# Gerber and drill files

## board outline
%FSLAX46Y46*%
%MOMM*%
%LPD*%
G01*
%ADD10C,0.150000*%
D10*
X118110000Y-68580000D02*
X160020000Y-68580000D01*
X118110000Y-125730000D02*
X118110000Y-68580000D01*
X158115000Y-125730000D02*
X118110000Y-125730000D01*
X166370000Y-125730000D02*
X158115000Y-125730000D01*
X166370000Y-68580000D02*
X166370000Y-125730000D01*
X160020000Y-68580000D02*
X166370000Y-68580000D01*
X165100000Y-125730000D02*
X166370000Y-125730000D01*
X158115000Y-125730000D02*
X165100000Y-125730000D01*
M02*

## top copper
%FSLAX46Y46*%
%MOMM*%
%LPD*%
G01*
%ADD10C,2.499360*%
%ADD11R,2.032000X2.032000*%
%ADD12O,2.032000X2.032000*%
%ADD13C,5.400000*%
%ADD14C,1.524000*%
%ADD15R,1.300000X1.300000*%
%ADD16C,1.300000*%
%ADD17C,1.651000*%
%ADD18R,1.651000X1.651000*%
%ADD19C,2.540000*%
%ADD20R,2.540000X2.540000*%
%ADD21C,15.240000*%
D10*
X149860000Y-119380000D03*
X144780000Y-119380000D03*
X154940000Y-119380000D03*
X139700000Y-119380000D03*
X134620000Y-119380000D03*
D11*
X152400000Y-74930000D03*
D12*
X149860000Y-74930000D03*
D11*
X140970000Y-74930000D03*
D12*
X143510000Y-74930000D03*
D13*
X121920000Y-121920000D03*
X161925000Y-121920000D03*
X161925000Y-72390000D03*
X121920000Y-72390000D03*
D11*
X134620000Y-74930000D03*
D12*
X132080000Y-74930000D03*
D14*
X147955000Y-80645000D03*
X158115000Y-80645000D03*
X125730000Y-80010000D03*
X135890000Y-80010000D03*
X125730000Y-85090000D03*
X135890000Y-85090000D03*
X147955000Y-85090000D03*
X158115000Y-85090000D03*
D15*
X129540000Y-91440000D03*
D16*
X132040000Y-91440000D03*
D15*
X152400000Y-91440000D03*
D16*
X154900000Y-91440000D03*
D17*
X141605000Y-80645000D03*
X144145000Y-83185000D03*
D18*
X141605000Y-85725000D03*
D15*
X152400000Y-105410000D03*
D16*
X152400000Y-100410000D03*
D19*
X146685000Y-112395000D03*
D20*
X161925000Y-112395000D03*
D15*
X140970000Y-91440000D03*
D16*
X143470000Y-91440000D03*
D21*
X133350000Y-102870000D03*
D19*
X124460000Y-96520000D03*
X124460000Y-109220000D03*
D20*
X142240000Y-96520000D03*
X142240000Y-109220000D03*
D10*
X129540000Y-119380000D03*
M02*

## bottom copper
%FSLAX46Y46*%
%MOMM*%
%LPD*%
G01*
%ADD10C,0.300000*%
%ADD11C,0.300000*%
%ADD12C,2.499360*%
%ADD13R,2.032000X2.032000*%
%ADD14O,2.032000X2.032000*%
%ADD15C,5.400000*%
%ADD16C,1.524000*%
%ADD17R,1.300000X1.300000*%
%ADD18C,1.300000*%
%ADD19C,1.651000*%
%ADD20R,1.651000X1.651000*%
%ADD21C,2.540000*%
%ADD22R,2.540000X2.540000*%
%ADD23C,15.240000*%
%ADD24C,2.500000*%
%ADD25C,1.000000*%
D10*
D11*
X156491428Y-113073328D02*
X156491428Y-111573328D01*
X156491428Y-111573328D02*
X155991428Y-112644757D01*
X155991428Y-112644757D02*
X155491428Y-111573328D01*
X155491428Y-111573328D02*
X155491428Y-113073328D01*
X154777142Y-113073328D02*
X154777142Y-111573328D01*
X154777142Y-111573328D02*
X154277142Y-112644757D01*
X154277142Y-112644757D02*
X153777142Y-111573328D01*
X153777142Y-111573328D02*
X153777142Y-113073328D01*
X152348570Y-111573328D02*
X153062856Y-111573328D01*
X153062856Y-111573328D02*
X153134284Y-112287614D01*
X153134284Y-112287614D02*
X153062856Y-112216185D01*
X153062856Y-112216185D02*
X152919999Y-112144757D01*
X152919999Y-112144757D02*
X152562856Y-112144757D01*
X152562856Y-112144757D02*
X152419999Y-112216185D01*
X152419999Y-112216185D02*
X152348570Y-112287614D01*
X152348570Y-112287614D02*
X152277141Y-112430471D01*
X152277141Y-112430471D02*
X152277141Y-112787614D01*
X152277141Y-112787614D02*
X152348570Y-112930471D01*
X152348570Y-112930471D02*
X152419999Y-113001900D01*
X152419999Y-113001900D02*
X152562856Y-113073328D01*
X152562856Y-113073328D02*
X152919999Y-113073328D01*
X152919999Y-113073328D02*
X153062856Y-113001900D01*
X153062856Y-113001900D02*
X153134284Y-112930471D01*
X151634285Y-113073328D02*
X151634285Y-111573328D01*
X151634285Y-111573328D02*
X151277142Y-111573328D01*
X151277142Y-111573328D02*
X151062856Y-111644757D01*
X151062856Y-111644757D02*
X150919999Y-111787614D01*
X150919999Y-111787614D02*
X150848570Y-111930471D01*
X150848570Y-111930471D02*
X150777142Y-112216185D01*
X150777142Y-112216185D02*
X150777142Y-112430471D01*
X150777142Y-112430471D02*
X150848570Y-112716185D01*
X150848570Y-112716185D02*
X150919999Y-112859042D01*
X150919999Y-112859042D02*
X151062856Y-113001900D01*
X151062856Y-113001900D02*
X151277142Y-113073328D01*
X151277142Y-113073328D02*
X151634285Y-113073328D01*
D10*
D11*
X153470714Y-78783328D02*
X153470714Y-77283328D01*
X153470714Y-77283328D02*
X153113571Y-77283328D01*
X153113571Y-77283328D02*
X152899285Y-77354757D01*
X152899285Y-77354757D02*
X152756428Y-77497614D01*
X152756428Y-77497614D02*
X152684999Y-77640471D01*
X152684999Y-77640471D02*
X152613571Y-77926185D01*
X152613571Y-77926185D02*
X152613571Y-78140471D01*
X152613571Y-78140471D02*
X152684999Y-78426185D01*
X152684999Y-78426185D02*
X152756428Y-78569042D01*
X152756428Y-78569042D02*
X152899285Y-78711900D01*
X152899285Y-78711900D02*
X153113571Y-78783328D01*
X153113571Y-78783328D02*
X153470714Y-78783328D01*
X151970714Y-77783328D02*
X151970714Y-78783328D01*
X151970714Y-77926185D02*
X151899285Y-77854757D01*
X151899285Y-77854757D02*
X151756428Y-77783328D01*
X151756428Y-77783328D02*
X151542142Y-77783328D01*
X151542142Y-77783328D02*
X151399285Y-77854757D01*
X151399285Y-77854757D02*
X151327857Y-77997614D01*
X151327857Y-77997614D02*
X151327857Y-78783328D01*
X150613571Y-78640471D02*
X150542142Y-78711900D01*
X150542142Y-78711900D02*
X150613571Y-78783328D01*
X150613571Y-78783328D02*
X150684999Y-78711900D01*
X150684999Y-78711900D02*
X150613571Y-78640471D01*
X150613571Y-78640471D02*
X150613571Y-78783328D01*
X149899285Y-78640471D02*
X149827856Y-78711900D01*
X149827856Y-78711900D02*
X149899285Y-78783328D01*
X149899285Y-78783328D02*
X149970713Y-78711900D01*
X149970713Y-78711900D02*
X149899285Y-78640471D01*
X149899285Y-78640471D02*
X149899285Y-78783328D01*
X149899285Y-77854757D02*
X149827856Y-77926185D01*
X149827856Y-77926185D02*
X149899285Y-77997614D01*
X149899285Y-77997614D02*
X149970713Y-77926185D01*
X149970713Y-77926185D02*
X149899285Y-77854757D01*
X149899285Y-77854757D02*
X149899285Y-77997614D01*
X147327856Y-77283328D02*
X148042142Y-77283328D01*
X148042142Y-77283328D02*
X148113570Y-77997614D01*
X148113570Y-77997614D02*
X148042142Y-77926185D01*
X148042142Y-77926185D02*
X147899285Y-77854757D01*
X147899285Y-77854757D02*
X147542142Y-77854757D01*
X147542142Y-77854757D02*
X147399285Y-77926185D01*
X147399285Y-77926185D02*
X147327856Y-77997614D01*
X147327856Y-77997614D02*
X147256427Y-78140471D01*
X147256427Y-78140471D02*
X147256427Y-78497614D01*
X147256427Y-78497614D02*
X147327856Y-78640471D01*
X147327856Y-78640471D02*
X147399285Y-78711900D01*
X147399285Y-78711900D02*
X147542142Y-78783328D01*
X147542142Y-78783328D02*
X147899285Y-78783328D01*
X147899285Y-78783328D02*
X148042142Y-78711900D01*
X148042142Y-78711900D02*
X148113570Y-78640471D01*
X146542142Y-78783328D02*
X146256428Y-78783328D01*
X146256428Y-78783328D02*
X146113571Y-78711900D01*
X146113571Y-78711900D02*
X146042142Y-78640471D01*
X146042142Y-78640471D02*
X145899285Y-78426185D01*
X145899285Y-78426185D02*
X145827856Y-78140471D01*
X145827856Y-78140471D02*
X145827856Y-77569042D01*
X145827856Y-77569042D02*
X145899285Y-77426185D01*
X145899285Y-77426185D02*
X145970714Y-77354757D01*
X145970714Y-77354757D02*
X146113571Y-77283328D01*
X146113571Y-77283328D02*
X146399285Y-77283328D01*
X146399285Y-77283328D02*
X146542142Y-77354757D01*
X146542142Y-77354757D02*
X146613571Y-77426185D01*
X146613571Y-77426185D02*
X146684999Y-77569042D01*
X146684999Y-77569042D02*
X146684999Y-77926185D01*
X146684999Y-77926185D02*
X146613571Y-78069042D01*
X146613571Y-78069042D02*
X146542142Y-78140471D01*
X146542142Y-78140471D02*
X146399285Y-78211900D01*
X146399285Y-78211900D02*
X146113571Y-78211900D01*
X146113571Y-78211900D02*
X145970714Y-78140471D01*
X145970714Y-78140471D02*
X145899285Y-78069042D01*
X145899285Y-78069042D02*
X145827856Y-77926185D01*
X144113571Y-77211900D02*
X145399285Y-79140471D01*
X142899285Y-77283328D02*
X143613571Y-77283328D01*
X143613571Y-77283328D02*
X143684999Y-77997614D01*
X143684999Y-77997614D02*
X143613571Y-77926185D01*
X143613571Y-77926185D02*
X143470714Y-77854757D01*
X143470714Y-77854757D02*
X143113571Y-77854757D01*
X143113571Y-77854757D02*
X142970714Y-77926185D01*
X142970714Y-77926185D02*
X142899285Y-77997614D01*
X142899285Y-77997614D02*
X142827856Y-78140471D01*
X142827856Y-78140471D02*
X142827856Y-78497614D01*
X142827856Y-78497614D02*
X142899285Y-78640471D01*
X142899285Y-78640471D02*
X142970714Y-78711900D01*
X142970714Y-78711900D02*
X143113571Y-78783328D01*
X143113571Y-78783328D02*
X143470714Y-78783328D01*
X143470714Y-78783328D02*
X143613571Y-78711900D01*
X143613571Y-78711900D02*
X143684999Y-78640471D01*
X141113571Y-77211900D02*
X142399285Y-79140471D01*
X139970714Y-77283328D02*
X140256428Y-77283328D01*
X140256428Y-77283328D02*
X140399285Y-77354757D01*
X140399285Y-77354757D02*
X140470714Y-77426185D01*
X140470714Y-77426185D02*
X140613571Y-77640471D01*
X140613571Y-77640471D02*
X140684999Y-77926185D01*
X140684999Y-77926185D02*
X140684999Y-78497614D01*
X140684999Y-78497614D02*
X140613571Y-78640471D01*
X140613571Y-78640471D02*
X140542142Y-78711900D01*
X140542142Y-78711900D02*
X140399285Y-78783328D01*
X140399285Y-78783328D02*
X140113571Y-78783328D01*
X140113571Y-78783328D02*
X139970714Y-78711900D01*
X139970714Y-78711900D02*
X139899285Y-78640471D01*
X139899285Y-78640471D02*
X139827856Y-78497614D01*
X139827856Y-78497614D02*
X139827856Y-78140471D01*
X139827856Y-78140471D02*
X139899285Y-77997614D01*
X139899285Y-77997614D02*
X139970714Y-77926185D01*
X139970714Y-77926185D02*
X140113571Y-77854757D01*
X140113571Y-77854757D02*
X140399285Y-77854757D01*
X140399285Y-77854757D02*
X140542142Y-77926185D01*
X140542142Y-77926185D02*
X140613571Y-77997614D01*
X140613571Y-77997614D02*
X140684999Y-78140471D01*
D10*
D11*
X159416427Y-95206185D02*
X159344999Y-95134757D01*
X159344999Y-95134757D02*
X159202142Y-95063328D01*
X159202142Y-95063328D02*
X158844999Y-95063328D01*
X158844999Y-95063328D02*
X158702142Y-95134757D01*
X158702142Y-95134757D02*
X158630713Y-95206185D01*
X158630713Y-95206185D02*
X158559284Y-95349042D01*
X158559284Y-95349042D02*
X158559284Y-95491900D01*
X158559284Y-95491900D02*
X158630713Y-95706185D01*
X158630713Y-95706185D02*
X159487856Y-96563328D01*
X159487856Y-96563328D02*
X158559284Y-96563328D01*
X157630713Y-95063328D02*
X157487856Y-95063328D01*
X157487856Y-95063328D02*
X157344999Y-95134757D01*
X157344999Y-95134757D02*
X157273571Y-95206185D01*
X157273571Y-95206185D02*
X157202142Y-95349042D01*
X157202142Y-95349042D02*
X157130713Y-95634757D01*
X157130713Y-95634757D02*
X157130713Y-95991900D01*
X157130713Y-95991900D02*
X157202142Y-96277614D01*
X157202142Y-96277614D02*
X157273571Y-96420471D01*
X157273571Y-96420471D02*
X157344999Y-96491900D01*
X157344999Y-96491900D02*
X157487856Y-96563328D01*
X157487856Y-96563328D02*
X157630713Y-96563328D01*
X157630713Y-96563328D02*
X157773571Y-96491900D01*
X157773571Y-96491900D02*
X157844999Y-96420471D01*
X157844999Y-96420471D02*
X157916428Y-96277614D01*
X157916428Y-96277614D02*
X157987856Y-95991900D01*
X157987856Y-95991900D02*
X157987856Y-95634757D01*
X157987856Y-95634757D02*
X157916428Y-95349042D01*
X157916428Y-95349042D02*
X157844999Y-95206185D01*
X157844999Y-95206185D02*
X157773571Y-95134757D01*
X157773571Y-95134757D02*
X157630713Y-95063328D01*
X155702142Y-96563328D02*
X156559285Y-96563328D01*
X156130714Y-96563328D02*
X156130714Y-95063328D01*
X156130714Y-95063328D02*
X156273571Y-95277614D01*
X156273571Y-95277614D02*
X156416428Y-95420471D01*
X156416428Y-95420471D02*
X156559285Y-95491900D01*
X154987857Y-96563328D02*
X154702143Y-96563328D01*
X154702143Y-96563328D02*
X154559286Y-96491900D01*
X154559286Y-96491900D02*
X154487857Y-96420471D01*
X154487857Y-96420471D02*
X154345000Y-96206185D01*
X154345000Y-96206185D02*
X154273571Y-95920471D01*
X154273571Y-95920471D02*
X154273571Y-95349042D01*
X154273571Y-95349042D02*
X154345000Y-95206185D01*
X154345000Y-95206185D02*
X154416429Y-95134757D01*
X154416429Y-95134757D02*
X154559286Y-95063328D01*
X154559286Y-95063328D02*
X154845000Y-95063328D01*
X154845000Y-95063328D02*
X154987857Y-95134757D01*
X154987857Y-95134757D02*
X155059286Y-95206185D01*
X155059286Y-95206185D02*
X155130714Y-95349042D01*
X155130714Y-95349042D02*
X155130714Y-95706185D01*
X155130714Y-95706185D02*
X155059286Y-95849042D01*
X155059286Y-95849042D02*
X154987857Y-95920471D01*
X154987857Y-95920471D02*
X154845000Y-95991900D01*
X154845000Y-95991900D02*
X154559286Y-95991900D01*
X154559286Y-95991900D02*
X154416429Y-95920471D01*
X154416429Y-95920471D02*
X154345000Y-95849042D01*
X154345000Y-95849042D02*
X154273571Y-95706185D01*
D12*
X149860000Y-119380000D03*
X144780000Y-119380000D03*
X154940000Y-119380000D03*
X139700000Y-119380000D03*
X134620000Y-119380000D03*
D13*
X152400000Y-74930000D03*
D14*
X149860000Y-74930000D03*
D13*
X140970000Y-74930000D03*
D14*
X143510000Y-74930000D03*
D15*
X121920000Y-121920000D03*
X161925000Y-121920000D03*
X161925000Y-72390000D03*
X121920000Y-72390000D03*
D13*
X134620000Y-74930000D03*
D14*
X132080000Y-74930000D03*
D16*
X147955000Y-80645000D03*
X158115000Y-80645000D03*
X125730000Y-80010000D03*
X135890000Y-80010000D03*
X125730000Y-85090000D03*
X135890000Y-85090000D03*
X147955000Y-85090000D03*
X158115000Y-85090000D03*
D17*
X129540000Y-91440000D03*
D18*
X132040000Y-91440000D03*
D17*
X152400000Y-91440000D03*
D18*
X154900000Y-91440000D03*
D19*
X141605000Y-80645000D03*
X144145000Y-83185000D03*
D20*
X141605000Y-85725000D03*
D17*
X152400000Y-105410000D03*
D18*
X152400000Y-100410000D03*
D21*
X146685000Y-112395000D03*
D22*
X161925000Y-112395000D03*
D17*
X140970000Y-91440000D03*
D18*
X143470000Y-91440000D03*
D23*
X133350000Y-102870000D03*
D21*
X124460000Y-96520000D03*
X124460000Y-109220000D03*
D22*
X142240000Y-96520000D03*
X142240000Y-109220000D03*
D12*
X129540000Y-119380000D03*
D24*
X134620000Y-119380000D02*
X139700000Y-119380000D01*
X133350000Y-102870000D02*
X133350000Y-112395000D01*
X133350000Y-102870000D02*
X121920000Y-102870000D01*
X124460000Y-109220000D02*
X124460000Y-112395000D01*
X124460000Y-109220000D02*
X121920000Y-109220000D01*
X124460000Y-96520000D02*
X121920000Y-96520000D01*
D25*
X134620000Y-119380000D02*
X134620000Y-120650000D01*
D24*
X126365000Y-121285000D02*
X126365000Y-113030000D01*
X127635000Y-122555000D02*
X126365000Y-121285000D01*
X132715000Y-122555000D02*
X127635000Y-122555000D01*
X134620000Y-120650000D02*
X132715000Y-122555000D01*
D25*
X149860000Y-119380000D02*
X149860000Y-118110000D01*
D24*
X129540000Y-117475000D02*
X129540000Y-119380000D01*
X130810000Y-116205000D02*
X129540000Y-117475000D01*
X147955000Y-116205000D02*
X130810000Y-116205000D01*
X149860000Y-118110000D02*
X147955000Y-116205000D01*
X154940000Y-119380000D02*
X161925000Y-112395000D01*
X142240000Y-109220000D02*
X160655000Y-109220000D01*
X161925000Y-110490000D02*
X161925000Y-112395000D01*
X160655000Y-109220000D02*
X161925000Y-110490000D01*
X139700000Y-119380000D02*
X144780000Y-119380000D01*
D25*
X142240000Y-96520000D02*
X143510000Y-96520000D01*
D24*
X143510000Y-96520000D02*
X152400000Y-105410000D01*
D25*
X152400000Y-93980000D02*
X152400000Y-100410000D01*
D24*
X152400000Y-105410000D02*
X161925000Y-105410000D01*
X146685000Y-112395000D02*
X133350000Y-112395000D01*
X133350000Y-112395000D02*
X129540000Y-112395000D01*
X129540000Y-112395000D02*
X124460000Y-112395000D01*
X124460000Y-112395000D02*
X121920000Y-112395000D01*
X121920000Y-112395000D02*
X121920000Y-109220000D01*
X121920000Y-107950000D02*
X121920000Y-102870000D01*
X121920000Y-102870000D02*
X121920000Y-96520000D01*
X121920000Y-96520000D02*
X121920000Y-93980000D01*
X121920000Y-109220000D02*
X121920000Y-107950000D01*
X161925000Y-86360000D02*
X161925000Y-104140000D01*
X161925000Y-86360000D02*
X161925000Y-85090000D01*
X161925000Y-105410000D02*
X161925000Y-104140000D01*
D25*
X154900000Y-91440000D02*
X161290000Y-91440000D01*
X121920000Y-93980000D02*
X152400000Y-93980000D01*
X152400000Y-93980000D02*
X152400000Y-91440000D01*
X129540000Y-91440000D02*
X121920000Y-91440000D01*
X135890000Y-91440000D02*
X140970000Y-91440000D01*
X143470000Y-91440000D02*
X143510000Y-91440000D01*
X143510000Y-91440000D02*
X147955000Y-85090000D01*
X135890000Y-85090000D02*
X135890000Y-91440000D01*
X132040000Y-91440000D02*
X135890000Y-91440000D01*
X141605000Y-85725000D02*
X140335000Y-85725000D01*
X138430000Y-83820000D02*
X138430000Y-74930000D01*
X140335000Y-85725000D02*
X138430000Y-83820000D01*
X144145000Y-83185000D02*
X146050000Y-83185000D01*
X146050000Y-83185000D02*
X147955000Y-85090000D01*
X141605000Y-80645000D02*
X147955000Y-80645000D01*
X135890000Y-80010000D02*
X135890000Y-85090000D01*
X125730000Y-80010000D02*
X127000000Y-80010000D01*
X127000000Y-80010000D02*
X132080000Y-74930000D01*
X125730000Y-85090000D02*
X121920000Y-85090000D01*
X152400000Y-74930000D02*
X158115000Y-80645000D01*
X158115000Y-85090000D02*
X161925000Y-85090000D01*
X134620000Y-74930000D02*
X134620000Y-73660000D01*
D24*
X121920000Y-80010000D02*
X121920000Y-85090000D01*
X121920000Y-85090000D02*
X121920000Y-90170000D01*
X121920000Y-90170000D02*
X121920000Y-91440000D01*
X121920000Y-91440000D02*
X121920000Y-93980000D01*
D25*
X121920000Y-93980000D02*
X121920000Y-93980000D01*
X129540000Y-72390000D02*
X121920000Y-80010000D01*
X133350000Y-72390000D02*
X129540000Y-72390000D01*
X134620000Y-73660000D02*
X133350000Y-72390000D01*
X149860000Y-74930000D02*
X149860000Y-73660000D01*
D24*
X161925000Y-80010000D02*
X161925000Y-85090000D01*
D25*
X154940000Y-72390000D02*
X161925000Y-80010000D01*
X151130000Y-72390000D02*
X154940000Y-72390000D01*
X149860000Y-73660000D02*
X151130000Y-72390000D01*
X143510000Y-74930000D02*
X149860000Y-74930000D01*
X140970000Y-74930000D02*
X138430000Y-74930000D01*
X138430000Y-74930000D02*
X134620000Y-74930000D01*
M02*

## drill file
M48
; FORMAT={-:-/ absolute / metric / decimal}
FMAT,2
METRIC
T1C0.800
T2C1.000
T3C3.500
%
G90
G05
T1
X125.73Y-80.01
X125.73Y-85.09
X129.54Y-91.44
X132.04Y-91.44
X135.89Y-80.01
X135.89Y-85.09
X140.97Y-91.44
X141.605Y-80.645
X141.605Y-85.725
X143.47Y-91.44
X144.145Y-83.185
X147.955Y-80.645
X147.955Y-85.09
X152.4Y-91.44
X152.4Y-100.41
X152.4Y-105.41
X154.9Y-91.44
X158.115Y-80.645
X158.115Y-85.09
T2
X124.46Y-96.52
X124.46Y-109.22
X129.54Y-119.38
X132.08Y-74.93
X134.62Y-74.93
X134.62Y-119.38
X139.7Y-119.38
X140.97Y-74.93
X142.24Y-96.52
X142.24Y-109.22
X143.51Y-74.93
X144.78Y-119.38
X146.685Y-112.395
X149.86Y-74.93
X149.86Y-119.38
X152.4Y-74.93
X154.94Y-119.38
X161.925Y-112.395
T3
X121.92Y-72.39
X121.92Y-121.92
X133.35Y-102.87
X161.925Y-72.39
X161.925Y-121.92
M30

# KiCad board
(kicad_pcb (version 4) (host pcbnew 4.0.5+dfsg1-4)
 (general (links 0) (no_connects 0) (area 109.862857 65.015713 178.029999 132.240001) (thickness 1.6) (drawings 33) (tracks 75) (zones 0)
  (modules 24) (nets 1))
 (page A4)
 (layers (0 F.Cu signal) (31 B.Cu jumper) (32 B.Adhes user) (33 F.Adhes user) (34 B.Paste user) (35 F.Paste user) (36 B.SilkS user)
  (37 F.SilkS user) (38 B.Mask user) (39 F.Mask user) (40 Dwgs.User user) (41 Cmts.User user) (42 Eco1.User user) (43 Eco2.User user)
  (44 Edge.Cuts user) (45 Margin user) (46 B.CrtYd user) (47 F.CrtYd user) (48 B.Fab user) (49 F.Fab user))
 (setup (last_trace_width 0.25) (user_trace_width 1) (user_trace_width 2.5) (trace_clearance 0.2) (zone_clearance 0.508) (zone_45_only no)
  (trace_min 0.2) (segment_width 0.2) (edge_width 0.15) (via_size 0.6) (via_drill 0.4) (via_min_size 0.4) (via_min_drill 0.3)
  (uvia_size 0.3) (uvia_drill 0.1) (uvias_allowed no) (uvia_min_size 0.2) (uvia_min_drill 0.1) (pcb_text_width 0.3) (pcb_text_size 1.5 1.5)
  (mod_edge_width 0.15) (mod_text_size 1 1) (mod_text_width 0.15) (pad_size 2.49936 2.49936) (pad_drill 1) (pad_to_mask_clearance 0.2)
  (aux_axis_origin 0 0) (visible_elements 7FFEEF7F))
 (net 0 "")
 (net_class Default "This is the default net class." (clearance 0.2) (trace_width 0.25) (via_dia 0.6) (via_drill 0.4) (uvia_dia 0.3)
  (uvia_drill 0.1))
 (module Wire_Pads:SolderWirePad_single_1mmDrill (layer F.Cu) (at 149.86 119.38)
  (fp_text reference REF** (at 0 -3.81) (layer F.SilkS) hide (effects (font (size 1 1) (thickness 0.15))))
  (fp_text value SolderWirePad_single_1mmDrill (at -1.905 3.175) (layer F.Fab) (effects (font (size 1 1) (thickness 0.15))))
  (pad 2 thru_hole circle (at 0 0) (size 2.49936 2.49936) (drill 1) (layers *.Cu *.Mask)))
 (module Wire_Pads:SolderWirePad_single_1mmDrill (layer F.Cu) (at 144.78 119.38)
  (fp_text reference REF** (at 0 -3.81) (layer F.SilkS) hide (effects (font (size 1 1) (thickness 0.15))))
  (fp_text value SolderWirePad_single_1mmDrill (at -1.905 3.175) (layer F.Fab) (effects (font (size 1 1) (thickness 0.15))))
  (pad 1 thru_hole circle (at 0 0) (size 2.49936 2.49936) (drill 1) (layers *.Cu *.Mask)))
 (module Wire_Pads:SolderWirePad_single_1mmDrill (layer F.Cu) (at 154.94 119.38)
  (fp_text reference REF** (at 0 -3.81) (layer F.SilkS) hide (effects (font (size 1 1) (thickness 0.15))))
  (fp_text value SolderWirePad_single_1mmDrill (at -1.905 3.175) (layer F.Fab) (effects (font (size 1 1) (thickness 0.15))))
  (pad 3 thru_hole circle (at 0 0) (size 2.49936 2.49936) (drill 1) (layers *.Cu *.Mask)))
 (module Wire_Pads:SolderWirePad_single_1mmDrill (layer F.Cu) (at 139.7 119.38)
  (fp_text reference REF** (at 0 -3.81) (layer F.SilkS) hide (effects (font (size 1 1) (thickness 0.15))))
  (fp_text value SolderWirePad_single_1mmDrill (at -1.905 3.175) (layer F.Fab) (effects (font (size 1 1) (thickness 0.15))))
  (pad 3 thru_hole circle (at 0 0) (size 2.49936 2.49936) (drill 1) (layers *.Cu *.Mask)))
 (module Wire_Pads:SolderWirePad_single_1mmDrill (layer F.Cu) (at 134.62 119.38)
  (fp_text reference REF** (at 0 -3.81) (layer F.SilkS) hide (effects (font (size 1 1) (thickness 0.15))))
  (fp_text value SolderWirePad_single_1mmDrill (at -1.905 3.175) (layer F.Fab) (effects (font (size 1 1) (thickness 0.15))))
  (pad 2 thru_hole circle (at 0 0) (size 2.49936 2.49936) (drill 1) (layers *.Cu *.Mask)))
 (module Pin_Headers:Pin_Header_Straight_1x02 (layer F.Cu) (at 152.4 74.93 270)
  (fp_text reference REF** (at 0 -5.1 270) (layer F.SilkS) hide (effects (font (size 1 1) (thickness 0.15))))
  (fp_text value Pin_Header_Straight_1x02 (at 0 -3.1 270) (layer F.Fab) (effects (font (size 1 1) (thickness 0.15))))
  (pad 1 thru_hole rect (at 0 0 270) (size 2.032 2.032) (drill 1) (layers *.Cu *.Mask))
  (pad 2 thru_hole oval (at 0 2.54 270) (size 2.032 2.032) (drill 1) (layers *.Cu *.Mask)))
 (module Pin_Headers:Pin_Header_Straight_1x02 (layer F.Cu) (at 140.97 74.93 90)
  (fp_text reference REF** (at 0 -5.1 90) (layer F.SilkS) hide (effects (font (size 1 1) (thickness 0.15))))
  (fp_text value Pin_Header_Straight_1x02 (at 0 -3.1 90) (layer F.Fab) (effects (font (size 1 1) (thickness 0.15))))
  (pad 1 thru_hole rect (at 0 0 90) (size 2.032 2.032) (drill 1) (layers *.Cu *.Mask))
  (pad 2 thru_hole oval (at 0 2.54 90) (size 2.032 2.032) (drill 1) (layers *.Cu *.Mask)))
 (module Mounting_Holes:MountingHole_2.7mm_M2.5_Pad (layer F.Cu) (at 121.92 121.92)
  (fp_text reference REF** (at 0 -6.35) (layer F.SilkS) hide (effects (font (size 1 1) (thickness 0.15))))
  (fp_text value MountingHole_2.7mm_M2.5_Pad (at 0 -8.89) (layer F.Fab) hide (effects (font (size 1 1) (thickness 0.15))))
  (pad 1 thru_hole circle (at 0 0) (size 5.4 5.4) (drill 3.5) (layers *.Cu *.Mask)))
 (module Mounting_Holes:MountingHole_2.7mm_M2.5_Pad (layer F.Cu) (at 161.925 121.92)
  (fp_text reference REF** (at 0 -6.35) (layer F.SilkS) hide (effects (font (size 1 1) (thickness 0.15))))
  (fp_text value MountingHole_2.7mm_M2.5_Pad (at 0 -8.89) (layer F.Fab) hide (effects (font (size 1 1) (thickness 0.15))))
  (pad 1 thru_hole circle (at 0 0) (size 5.4 5.4) (drill 3.5) (layers *.Cu *.Mask)))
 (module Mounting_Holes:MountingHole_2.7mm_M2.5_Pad (layer F.Cu) (at 161.925 72.39)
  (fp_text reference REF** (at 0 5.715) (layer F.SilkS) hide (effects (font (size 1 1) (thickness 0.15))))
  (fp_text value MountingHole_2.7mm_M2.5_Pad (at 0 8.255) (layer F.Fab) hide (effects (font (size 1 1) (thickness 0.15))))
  (pad 1 thru_hole circle (at 0 0) (size 5.4 5.4) (drill 3.5) (layers *.Cu *.Mask)))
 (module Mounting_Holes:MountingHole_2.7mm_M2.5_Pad (layer F.Cu) (at 121.92 72.39)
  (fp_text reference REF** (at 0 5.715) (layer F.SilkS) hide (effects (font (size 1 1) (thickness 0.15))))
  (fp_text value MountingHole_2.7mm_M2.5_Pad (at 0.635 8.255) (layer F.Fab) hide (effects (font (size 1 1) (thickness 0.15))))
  (pad 1 thru_hole circle (at 0 0) (size 5.4 5.4) (drill 3.5) (layers *.Cu *.Mask)))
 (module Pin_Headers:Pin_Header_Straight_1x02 (layer F.Cu) (at 134.62 74.93 270)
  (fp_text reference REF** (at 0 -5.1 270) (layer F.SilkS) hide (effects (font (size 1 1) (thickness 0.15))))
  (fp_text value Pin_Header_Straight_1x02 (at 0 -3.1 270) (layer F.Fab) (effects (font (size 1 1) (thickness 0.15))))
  (pad 1 thru_hole rect (at 0 0 270) (size 2.032 2.032) (drill 1) (layers *.Cu *.Mask))
  (pad 2 thru_hole oval (at 0 2.54 270) (size 2.032 2.032) (drill 1) (layers *.Cu *.Mask)))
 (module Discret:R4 (layer F.Cu) (at 153.035 80.645)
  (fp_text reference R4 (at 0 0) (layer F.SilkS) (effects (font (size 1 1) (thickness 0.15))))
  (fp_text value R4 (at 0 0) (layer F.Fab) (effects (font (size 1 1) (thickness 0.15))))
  (pad 1 thru_hole circle (at -5.08 0) (size 1.524 1.524) (drill 0.8) (layers *.Cu *.Mask))
  (pad 2 thru_hole circle (at 5.08 0) (size 1.524 1.524) (drill 0.8) (layers *.Cu *.Mask)))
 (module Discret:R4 (layer F.Cu) (at 130.81 80.01)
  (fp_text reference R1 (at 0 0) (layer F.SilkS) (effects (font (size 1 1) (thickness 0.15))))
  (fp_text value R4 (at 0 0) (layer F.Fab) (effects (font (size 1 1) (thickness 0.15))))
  (pad 1 thru_hole circle (at -5.08 0) (size 1.524 1.524) (drill 0.8) (layers *.Cu *.Mask))
  (pad 2 thru_hole circle (at 5.08 0) (size 1.524 1.524) (drill 0.8) (layers *.Cu *.Mask)))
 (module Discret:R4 (layer F.Cu) (at 130.81 85.09)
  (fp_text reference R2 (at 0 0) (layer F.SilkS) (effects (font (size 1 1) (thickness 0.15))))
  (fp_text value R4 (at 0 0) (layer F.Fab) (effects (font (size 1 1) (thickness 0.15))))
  (pad 1 thru_hole circle (at -5.08 0) (size 1.524 1.524) (drill 0.8) (layers *.Cu *.Mask))
  (pad 2 thru_hole circle (at 5.08 0) (size 1.524 1.524) (drill 0.8) (layers *.Cu *.Mask)))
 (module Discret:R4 (layer F.Cu) (at 153.035 85.09)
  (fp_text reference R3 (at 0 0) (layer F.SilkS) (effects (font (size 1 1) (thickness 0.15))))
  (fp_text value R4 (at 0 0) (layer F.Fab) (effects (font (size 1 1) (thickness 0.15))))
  (pad 1 thru_hole circle (at -5.08 0) (size 1.524 1.524) (drill 0.8) (layers *.Cu *.Mask))
  (pad 2 thru_hole circle (at 5.08 0) (size 1.524 1.524) (drill 0.8) (layers *.Cu *.Mask)))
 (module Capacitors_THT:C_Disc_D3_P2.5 (layer F.Cu) (at 129.54 91.44)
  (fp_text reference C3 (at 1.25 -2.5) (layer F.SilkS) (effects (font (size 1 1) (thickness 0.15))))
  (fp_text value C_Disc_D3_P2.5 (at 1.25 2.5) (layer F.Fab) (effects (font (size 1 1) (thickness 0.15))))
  (pad 1 thru_hole rect (at 0 0) (size 1.3 1.3) (drill 0.8) (layers *.Cu *.Mask))
  (pad 2 thru_hole circle (at 2.5 0) (size 1.3 1.3) (drill 0.8) (layers *.Cu *.Mask)))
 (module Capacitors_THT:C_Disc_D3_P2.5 (layer F.Cu) (at 152.4 91.44)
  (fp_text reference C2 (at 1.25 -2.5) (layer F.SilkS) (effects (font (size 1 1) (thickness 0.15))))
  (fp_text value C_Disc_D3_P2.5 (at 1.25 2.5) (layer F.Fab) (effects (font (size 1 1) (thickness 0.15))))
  (pad 1 thru_hole rect (at 0 0) (size 1.3 1.3) (drill 0.8) (layers *.Cu *.Mask))
  (pad 2 thru_hole circle (at 2.5 0) (size 1.3 1.3) (drill 0.8) (layers *.Cu *.Mask)))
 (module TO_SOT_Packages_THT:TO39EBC (layer F.Cu) (at 141.605 85.725 90)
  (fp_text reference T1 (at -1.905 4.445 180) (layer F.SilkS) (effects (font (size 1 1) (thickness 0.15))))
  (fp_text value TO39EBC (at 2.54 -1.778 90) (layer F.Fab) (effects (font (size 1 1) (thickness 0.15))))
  (pad 3 thru_hole circle (at 5.08 0 90) (size 1.651 1.651) (drill 0.8) (layers *.Cu *.Mask))
  (pad 2 thru_hole circle (at 2.54 2.54 90) (size 1.651 1.651) (drill 0.8) (layers *.Cu *.Mask))
  (pad 1 thru_hole rect (at 0 0 90) (size 1.651 1.651) (drill 0.8) (layers *.Cu *.Mask)))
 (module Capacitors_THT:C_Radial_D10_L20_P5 (layer F.Cu) (at 152.4 105.41 90)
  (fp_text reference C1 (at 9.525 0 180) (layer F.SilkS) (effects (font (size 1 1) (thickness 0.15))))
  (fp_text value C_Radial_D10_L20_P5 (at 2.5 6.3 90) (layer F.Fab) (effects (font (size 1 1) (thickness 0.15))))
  (pad 1 thru_hole rect (at 0 0 90) (size 1.3 1.3) (drill 0.8) (layers *.Cu *.Mask))
  (pad 2 thru_hole circle (at 5 0 90) (size 1.3 1.3) (drill 0.8) (layers *.Cu *.Mask)))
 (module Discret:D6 (layer F.Cu) (at 154.305 112.395)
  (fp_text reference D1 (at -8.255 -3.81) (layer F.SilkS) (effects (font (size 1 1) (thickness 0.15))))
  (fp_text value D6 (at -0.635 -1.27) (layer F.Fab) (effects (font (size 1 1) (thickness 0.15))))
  (pad 2 thru_hole circle (at -7.62 0) (size 2.54 2.54) (drill 1) (layers *.Cu *.Mask))
  (pad 1 thru_hole rect (at 7.62 0) (size 2.54 2.54) (drill 1) (layers *.Cu *.Mask)))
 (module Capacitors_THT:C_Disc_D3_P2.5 (layer F.Cu) (at 140.97 91.44)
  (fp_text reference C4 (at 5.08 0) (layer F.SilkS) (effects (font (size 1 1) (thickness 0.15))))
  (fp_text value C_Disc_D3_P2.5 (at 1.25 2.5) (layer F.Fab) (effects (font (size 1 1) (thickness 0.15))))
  (pad 1 thru_hole rect (at 0 0) (size 1.3 1.3) (drill 0.8) (layers *.Cu *.Mask))
  (pad 2 thru_hole circle (at 2.5 0) (size 1.3 1.3) (drill 0.8) (layers *.Cu *.Mask)))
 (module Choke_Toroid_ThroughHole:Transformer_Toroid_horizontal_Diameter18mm (layer F.Cu) (at 133.35 102.87)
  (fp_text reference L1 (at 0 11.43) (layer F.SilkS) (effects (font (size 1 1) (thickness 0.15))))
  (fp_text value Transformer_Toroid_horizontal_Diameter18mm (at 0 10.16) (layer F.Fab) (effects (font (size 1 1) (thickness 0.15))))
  (pad "" thru_hole circle (at 0 0) (size 15.24 15.24) (drill 3.5) (layers *.Cu *.SilkS *.Mask))
  (pad 1 thru_hole circle (at -8.89 -6.35) (size 2.54 2.54) (drill 1) (layers *.Cu *.SilkS *.Mask))
  (pad 2 thru_hole circle (at -8.89 6.35) (size 2.54 2.54) (drill 1) (layers *.Cu *.SilkS *.Mask))
  (pad 3 thru_hole rect (at 8.89 -6.35) (size 2.54 2.54) (drill 1) (layers *.Cu *.SilkS *.Mask))
  (pad 4 thru_hole rect (at 8.89 6.35) (size 2.54 2.54) (drill 1) (layers *.Cu *.SilkS *.Mask)))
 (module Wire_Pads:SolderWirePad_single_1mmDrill (layer F.Cu) (at 129.54 119.38)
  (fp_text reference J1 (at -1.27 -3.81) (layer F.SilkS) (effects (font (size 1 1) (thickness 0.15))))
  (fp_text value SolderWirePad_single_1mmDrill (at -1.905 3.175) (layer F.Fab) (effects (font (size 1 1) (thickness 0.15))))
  (pad 1 thru_hole circle (at 0 0) (size 2.49936 2.49936) (drill 1) (layers *.Cu *.Mask)))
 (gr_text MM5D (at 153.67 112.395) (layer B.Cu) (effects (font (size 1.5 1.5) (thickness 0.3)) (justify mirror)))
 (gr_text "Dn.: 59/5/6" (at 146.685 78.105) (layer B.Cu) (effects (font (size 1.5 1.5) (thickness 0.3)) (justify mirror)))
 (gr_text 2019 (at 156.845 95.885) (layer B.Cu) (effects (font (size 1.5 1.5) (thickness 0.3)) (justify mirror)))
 (gr_line (start 118.11 68.58) (end 160.02 68.58) (angle 90) (layer Edge.Cuts) (width 0.15))
 (gr_line (start 118.11 125.73) (end 118.11 68.58) (angle 90) (layer Edge.Cuts) (width 0.15))
 (gr_line (start 158.115 125.73) (end 118.11 125.73) (angle 90) (layer Edge.Cuts) (width 0.15))
 (gr_line (start 166.37 125.73) (end 158.115 125.73) (angle 90) (layer Edge.Cuts) (width 0.15))
 (gr_line (start 166.37 68.58) (end 166.37 125.73) (angle 90) (layer Edge.Cuts) (width 0.15))
 (gr_line (start 160.02 68.58) (end 166.37 68.58) (angle 90) (layer Edge.Cuts) (width 0.15))
 (gr_line (start 165.1 125.73) (end 166.37 125.73) (angle 90) (layer Edge.Cuts) (width 0.15))
 (gr_line (start 158.115 125.73) (end 165.1 125.73) (angle 90) (layer Edge.Cuts) (width 0.15))
 (segment (start 134.62 119.38) (end 139.7 119.38) (width 2.5) (layer B.Cu) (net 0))
 (segment (start 133.35 102.87) (end 133.35 112.395) (width 2.5) (layer B.Cu) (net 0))
 (segment (start 133.35 102.87) (end 121.92 102.87) (width 2.5) (layer B.Cu) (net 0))
 (segment (start 124.46 109.22) (end 124.46 112.395) (width 2.5) (layer B.Cu) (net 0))
 (segment (start 124.46 109.22) (end 121.92 109.22) (width 2.5) (layer B.Cu) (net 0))
 (segment (start 124.46 96.52) (end 121.92 96.52) (width 2.5) (layer B.Cu) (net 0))
 (segment (start 134.62 119.38) (end 134.62 120.65) (width 1) (layer B.Cu) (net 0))
 (segment (start 126.365 121.285) (end 126.365 113.03) (width 2.5) (layer B.Cu) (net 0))
 (segment (start 127.635 122.555) (end 126.365 121.285) (width 2.5) (layer B.Cu) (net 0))
 (segment (start 132.715 122.555) (end 127.635 122.555) (width 2.5) (layer B.Cu) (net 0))
 (segment (start 134.62 120.65) (end 132.715 122.555) (width 2.5) (layer B.Cu) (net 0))
 (segment (start 149.86 119.38) (end 149.86 118.11) (width 1) (layer B.Cu) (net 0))
 (segment (start 129.54 117.475) (end 129.54 119.38) (width 2.5) (layer B.Cu) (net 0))
 (segment (start 130.81 116.205) (end 129.54 117.475) (width 2.5) (layer B.Cu) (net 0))
 (segment (start 147.955 116.205) (end 130.81 116.205) (width 2.5) (layer B.Cu) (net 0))
 (segment (start 149.86 118.11) (end 147.955 116.205) (width 2.5) (layer B.Cu) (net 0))
 (segment (start 154.94 119.38) (end 161.925 112.395) (width 2.5) (layer B.Cu) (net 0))
 (segment (start 142.24 109.22) (end 160.655 109.22) (width 2.5) (layer B.Cu) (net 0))
 (segment (start 161.925 110.49) (end 161.925 112.395) (width 2.5) (layer B.Cu) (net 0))
 (segment (start 160.655 109.22) (end 161.925 110.49) (width 2.5) (layer B.Cu) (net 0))
 (segment (start 139.7 119.38) (end 144.78 119.38) (width 2.5) (layer B.Cu) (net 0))
 (segment (start 142.24 96.52) (end 143.51 96.52) (width 1) (layer B.Cu) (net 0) (status 30))
 (segment (start 143.51 96.52) (end 152.4 105.41) (width 2.5) (layer B.Cu) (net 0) (status 20))
 (segment (start 152.4 93.98) (end 152.4 100.41) (width 1) (layer B.Cu) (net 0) (status 20))
 (segment (start 152.4 105.41) (end 161.925 105.41) (width 2.5) (layer B.Cu) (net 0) (status 10))
 (segment (start 146.685 112.395) (end 133.35 112.395) (width 2.5) (layer B.Cu) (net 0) (status 10))
 (segment (start 133.35 112.395) (end 129.54 112.395) (width 2.5) (layer B.Cu) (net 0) (status 10))
 (segment (start 129.54 112.395) (end 124.46 112.395) (width 2.5) (layer B.Cu) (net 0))
 (segment (start 124.46 112.395) (end 121.92 112.395) (width 2.5) (layer B.Cu) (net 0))
 (segment (start 121.92 112.395) (end 121.92 109.22) (width 2.5) (layer B.Cu) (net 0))
 (segment (start 121.92 107.95) (end 121.92 102.87) (width 2.5) (layer B.Cu) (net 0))
 (segment (start 121.92 102.87) (end 121.92 96.52) (width 2.5) (layer B.Cu) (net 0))
 (segment (start 121.92 96.52) (end 121.92 93.98) (width 2.5) (layer B.Cu) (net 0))
 (segment (start 121.92 109.22) (end 121.92 107.95) (width 2.5) (layer B.Cu) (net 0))
 (segment (start 161.925 86.36) (end 161.925 104.14) (width 2.5) (layer B.Cu) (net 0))
 (segment (start 161.925 86.36) (end 161.925 85.09) (width 2.5) (layer B.Cu) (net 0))
 (segment (start 161.925 105.41) (end 161.925 104.14) (width 2.5) (layer B.Cu) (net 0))
 (segment (start 154.9 91.44) (end 161.29 91.44) (width 1) (layer B.Cu) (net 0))
 (segment (start 121.92 93.98) (end 152.4 93.98) (width 1) (layer B.Cu) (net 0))
 (segment (start 152.4 93.98) (end 152.4 91.44) (width 1) (layer B.Cu) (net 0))
 (segment (start 129.54 91.44) (end 121.92 91.44) (width 1) (layer B.Cu) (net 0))
 (segment (start 135.89 91.44) (end 140.97 91.44) (width 1) (layer B.Cu) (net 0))
 (segment (start 143.47 91.44) (end 143.51 91.44) (width 1) (layer B.Cu) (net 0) (status 30))
 (segment (start 143.51 91.44) (end 147.955 85.09) (width 1) (layer B.Cu) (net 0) (status 10))
 (segment (start 135.89 85.09) (end 135.89 91.44) (width 1) (layer B.Cu) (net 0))
 (segment (start 132.04 91.44) (end 135.89 91.44) (width 1) (layer B.Cu) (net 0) (status 10))
 (segment (start 141.605 85.725) (end 140.335 85.725) (width 1) (layer B.Cu) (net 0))
 (segment (start 138.43 83.82) (end 138.43 74.93) (width 1) (layer B.Cu) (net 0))
 (segment (start 140.335 85.725) (end 138.43 83.82) (width 1) (layer B.Cu) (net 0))
 (segment (start 144.145 83.185) (end 146.05 83.185) (width 1) (layer B.Cu) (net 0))
 (segment (start 146.05 83.185) (end 147.955 85.09) (width 1) (layer B.Cu) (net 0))
 (segment (start 141.605 80.645) (end 147.955 80.645) (width 1) (layer B.Cu) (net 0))
 (segment (start 135.89 80.01) (end 135.89 85.09) (width 1) (layer B.Cu) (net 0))
 (segment (start 125.73 80.01) (end 127 80.01) (width 1) (layer B.Cu) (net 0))
 (segment (start 127 80.01) (end 132.08 74.93) (width 1) (layer B.Cu) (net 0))
 (segment (start 125.73 85.09) (end 121.92 85.09) (width 1) (layer B.Cu) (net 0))
 (segment (start 152.4 74.93) (end 158.115 80.645) (width 1) (layer B.Cu) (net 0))
 (segment (start 158.115 85.09) (end 161.925 85.09) (width 1) (layer B.Cu) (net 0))
 (segment (start 134.62 74.93) (end 134.62 73.66) (width 1) (layer B.Cu) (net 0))
 (segment (start 121.92 80.01) (end 121.92 85.09) (width 2.5) (layer B.Cu) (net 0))
 (segment (start 121.92 85.09) (end 121.92 90.17) (width 2.5) (layer B.Cu) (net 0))
 (segment (start 121.92 90.17) (end 121.92 91.44) (width 2.5) (layer B.Cu) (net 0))
 (segment (start 121.92 91.44) (end 121.92 93.98) (width 2.5) (layer B.Cu) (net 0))
 (segment (start 121.92 93.98) (end 121.92 93.98) (width 1) (layer B.Cu) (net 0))
 (segment (start 129.54 72.39) (end 121.92 80.01) (width 1) (layer B.Cu) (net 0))
 (segment (start 133.35 72.39) (end 129.54 72.39) (width 1) (layer B.Cu) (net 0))
 (segment (start 134.62 73.66) (end 133.35 72.39) (width 1) (layer B.Cu) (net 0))
 (segment (start 149.86 74.93) (end 149.86 73.66) (width 1) (layer B.Cu) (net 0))
 (segment (start 161.925 80.01) (end 161.925 85.09) (width 2.5) (layer B.Cu) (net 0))
 (segment (start 154.94 72.39) (end 161.925 80.01) (width 1) (layer B.Cu) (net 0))
 (segment (start 151.13 72.39) (end 154.94 72.39) (width 1) (layer B.Cu) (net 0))
 (segment (start 149.86 73.66) (end 151.13 72.39) (width 1) (layer B.Cu) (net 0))
 (segment (start 143.51 74.93) (end 149.86 74.93) (width 1) (layer B.Cu) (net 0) (status 20))
 (segment (start 140.97 74.93) (end 138.43 74.93) (width 1) (layer B.Cu) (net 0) (status 20))
 (segment (start 138.43 74.93) (end 134.62 74.93) (width 1) (layer B.Cu) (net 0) (status 20)))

